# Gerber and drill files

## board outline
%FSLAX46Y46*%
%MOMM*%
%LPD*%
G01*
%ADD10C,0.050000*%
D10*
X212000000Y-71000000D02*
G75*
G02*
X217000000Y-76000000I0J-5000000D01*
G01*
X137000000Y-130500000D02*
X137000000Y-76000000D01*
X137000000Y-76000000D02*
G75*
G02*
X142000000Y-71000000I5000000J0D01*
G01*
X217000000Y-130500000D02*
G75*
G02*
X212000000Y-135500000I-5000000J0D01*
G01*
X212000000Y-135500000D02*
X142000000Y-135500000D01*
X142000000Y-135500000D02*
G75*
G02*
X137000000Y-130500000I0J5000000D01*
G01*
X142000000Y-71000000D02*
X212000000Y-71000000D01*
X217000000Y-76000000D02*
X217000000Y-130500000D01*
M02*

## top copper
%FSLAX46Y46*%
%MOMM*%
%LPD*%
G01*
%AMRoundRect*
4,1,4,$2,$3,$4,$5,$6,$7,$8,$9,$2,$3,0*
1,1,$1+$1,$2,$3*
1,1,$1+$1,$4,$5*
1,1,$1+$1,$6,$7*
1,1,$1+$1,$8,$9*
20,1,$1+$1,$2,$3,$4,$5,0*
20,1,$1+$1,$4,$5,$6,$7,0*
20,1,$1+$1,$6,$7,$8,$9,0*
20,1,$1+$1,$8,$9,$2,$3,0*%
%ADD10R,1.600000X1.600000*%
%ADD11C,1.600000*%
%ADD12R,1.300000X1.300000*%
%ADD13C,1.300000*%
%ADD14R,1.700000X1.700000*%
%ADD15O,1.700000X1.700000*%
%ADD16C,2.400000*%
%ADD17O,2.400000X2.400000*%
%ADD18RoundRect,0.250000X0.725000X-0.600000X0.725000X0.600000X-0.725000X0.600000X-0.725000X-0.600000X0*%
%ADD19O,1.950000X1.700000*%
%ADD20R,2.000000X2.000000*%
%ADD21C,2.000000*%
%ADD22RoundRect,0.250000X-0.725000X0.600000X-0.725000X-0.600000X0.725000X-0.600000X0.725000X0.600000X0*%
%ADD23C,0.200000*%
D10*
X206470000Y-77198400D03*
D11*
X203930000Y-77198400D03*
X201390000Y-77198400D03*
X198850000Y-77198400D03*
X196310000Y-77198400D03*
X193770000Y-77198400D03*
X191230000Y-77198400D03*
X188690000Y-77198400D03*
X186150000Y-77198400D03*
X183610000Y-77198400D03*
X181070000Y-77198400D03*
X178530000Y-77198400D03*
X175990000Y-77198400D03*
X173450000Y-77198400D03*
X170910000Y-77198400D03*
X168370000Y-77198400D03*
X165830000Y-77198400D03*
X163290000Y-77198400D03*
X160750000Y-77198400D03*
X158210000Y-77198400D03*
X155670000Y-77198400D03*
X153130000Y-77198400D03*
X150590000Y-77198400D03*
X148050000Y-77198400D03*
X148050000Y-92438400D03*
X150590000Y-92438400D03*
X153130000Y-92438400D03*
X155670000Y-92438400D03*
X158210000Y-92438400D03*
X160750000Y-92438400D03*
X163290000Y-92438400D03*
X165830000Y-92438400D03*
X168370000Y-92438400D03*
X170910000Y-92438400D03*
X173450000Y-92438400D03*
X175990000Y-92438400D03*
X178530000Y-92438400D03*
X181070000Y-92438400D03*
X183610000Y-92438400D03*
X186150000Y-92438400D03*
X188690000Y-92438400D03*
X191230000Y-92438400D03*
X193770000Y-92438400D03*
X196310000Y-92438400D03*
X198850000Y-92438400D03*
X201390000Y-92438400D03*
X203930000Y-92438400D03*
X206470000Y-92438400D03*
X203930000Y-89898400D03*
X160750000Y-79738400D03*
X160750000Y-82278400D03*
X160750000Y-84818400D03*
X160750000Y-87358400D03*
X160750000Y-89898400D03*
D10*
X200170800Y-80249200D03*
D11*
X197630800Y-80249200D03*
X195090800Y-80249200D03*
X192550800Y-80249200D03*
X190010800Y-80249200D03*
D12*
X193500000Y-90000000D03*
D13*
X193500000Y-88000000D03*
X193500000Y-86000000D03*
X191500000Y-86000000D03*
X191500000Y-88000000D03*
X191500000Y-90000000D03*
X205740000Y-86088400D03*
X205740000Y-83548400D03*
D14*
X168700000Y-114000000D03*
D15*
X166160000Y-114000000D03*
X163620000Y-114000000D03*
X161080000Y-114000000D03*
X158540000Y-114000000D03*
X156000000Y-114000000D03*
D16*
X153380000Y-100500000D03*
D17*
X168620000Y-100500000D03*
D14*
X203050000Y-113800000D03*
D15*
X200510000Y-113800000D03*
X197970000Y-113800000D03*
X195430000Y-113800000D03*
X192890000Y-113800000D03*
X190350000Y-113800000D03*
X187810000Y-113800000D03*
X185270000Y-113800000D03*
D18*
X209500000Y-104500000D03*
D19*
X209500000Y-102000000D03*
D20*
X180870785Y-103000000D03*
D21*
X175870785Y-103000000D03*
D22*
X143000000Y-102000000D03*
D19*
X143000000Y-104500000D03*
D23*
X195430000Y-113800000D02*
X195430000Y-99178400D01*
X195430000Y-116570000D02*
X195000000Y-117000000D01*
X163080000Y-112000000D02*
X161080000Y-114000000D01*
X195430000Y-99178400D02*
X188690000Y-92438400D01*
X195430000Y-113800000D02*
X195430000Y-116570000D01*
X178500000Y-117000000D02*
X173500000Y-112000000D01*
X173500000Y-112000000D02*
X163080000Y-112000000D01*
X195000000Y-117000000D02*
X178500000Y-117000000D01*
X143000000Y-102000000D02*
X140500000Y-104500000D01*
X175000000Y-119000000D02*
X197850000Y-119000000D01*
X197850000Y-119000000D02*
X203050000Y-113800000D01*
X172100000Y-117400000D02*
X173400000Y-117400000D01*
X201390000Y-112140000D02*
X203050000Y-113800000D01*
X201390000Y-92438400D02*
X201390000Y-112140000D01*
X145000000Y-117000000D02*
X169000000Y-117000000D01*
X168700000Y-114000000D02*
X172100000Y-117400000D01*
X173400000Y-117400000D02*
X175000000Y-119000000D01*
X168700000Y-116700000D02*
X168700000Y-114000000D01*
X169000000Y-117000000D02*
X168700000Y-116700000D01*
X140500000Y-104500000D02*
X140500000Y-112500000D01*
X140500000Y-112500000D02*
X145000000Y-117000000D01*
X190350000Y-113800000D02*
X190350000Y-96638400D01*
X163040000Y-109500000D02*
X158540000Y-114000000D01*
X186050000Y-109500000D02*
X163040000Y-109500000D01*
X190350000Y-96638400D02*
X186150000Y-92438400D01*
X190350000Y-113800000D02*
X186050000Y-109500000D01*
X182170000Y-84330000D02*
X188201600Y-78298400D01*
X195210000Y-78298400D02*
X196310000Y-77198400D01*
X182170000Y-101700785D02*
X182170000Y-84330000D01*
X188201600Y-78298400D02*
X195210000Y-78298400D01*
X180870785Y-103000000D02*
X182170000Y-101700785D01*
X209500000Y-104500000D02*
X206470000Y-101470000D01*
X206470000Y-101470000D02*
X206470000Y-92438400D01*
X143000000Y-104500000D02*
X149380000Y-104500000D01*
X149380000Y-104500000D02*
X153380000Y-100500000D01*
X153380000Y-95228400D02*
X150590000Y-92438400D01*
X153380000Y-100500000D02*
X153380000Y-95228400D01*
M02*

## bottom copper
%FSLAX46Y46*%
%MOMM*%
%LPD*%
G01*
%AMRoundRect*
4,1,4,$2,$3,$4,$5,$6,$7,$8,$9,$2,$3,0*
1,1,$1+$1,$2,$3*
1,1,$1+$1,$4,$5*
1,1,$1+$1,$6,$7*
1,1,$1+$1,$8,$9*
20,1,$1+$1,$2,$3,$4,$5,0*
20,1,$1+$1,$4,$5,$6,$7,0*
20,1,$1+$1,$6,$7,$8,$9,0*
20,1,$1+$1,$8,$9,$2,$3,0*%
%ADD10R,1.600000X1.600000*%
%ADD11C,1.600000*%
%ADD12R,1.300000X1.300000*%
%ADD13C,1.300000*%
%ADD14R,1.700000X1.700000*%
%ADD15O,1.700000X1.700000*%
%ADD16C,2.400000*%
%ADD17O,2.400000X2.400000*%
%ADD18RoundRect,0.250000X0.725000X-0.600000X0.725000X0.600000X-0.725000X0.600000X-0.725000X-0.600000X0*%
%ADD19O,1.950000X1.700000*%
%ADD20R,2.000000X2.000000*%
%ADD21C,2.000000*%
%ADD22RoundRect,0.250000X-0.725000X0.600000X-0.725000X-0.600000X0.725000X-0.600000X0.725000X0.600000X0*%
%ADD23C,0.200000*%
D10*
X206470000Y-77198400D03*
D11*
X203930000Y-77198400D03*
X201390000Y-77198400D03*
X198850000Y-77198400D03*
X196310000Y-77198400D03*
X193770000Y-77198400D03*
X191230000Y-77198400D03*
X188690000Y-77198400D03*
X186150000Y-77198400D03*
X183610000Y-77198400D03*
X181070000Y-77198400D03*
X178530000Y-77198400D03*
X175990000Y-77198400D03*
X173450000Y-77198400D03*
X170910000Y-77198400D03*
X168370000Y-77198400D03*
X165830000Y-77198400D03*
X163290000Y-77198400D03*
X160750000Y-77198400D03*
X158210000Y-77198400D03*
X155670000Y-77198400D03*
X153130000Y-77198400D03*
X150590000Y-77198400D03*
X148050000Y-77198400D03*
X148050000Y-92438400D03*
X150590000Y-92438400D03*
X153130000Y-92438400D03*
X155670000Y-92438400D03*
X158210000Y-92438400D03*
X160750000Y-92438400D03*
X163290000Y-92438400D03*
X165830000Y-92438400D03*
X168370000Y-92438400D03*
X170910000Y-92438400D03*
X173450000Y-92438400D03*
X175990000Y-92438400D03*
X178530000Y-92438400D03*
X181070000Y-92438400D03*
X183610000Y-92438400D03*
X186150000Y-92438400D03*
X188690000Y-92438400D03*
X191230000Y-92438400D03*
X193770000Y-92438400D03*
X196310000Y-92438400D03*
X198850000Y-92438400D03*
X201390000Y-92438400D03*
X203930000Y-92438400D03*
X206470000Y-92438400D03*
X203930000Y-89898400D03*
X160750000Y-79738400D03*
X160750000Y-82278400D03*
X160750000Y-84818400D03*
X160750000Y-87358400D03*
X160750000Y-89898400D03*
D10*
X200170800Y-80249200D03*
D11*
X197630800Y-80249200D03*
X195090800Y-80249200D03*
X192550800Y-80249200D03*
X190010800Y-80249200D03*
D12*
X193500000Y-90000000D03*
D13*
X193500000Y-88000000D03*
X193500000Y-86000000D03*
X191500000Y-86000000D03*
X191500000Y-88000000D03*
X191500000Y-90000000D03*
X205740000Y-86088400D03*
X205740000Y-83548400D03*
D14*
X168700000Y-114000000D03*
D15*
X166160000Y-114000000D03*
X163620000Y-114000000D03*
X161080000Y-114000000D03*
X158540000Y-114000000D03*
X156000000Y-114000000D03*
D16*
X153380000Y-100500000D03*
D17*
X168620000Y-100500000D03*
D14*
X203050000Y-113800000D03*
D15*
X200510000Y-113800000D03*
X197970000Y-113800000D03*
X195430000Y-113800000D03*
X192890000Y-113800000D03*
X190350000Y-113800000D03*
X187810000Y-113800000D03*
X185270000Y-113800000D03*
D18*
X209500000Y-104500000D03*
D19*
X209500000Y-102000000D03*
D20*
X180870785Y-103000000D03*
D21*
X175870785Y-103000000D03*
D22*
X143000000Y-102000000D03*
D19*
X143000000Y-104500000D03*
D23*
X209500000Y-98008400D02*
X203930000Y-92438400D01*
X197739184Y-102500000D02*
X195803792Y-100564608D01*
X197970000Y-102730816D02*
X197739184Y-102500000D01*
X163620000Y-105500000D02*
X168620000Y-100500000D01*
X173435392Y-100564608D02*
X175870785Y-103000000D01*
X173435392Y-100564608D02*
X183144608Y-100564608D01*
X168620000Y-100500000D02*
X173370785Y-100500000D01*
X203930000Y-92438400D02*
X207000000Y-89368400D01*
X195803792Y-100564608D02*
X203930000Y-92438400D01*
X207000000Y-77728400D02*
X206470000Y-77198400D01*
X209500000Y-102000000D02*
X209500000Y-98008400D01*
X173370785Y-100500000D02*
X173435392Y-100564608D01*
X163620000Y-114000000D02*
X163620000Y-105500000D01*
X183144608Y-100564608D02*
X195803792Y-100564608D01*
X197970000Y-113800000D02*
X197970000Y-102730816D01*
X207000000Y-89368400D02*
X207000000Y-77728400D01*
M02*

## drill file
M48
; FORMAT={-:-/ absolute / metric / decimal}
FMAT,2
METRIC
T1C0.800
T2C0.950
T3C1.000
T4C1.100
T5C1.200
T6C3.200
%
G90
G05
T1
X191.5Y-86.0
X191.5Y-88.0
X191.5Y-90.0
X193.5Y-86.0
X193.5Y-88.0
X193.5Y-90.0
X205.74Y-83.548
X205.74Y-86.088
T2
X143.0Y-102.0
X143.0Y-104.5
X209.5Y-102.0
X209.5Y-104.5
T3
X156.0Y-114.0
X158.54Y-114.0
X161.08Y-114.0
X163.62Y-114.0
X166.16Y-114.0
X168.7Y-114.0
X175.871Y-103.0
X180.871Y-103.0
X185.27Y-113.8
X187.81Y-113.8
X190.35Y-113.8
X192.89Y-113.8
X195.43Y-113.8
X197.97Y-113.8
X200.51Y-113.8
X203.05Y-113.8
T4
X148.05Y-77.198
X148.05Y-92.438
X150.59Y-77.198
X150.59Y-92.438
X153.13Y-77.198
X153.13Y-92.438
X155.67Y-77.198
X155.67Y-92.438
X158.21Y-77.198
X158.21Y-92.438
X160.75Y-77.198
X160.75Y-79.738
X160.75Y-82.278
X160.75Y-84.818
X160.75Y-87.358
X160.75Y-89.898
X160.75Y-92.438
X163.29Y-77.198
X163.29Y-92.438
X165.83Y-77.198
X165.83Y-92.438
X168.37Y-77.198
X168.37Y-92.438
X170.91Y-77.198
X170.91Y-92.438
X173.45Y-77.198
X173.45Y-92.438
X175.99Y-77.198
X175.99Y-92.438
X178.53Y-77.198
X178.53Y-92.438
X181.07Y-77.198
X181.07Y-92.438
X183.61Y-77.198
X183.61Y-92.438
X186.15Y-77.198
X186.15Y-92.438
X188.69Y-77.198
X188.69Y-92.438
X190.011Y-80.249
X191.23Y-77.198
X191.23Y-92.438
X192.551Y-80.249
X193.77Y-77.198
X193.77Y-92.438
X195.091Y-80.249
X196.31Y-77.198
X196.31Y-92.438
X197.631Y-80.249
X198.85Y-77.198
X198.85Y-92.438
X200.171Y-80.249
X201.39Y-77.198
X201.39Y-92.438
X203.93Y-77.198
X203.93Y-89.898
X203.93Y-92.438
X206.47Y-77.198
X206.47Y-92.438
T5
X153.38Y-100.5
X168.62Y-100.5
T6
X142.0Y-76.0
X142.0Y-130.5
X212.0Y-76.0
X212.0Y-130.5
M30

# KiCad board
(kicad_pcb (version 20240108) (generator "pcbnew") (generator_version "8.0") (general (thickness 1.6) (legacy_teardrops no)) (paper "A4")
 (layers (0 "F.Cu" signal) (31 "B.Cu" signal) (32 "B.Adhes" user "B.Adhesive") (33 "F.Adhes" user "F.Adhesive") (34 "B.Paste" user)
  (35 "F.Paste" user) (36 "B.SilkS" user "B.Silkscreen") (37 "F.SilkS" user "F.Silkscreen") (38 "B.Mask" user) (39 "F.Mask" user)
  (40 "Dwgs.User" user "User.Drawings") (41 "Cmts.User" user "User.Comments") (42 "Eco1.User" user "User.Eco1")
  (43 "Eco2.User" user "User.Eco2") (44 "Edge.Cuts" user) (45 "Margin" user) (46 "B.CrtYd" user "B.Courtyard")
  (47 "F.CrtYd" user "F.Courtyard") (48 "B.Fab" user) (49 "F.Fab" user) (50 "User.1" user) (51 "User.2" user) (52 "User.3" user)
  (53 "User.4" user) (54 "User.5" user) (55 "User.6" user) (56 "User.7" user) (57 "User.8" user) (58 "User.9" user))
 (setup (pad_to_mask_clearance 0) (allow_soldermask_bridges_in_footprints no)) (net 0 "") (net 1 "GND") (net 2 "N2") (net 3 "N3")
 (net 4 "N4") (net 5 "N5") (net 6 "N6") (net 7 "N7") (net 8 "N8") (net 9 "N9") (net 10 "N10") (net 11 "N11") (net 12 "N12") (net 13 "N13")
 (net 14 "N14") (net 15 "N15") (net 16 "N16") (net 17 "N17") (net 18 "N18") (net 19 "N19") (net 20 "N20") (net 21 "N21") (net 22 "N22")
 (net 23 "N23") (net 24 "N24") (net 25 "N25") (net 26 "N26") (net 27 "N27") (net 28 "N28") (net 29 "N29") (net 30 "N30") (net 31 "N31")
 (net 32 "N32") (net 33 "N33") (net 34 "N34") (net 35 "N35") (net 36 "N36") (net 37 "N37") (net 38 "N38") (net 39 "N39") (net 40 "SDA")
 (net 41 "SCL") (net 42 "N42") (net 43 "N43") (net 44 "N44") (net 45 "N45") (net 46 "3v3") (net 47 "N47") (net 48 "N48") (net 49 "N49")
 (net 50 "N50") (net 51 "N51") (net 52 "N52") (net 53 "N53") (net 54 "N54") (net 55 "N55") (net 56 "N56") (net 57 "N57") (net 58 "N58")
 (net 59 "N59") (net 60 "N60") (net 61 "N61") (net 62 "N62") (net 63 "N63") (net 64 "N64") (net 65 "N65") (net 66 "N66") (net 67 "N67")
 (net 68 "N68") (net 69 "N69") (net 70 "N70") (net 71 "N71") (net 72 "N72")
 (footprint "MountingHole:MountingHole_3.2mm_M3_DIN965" (layer "F.Cu") (at 212 76)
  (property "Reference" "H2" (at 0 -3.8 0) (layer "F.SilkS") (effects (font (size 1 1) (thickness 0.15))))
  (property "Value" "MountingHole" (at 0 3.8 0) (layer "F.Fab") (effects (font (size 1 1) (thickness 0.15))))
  (pad "" np_thru_hole circle (at 0 0) (size 3.2 3.2) (drill 3.2) (layers "*.Cu" "*.Mask")))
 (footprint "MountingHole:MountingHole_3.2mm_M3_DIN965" (layer "F.Cu") (at 142 76)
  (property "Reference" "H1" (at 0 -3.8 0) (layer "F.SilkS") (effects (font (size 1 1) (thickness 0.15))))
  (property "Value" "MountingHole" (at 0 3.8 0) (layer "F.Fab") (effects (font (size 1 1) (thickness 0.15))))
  (pad "" np_thru_hole circle (at 0 0) (size 3.2 3.2) (drill 3.2) (layers "*.Cu" "*.Mask")))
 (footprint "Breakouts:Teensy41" (layer "F.Cu") (at 177.26 84.8184 180)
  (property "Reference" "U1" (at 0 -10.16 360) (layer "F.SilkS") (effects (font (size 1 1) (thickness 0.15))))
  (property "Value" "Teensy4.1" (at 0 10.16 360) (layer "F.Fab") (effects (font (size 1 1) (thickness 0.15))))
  (pad "1" thru_hole rect (at -29.21 7.62 180) (size 1.6 1.6) (drill 1.1) (layers "*.Cu" "*.Mask") (remove_unused_layers no) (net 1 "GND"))
  (pad "2" thru_hole circle (at -26.67 7.62 180) (size 1.6 1.6) (drill 1.1) (layers "*.Cu" "*.Mask") (remove_unused_layers no) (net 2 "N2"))
  (pad "3" thru_hole circle (at -24.13 7.62 180) (size 1.6 1.6) (drill 1.1) (layers "*.Cu" "*.Mask") (remove_unused_layers no) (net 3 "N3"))
  (pad "4" thru_hole circle (at -21.59 7.62 180) (size 1.6 1.6) (drill 1.1) (layers "*.Cu" "*.Mask") (remove_unused_layers no) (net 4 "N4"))
  (pad "5" thru_hole circle (at -19.05 7.62 180) (size 1.6 1.6) (drill 1.1) (layers "*.Cu" "*.Mask") (remove_unused_layers no) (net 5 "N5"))
  (pad "6" thru_hole circle (at -16.51 7.62 180) (size 1.6 1.6) (drill 1.1) (layers "*.Cu" "*.Mask") (remove_unused_layers no) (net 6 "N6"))
  (pad "7" thru_hole circle (at -13.97 7.62 180) (size 1.6 1.6) (drill 1.1) (layers "*.Cu" "*.Mask") (remove_unused_layers no) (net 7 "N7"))
  (pad "8" thru_hole circle (at -11.43 7.62 180) (size 1.6 1.6) (drill 1.1) (layers "*.Cu" "*.Mask") (remove_unused_layers no) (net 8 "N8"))
  (pad "9" thru_hole circle (at -8.89 7.62 180) (size 1.6 1.6) (drill 1.1) (layers "*.Cu" "*.Mask") (remove_unused_layers no) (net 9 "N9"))
  (pad "10" thru_hole circle (at -6.35 7.62 180) (size 1.6 1.6) (drill 1.1) (layers "*.Cu" "*.Mask") (remove_unused_layers no)
   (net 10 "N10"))
  (pad "11" thru_hole circle (at -3.81 7.62 180) (size 1.6 1.6) (drill 1.1) (layers "*.Cu" "*.Mask") (remove_unused_layers no)
   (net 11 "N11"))
  (pad "12" thru_hole circle (at -1.27 7.62 180) (size 1.6 1.6) (drill 1.1) (layers "*.Cu" "*.Mask") (remove_unused_layers no)
   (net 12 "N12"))
  (pad "13" thru_hole circle (at 1.27 7.62 180) (size 1.6 1.6) (drill 1.1) (layers "*.Cu" "*.Mask") (remove_unused_layers no) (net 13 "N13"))
  (pad "14" thru_hole circle (at 3.81 7.62 180) (size 1.6 1.6) (drill 1.1) (layers "*.Cu" "*.Mask") (remove_unused_layers no) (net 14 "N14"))
  (pad "15" thru_hole circle (at 6.35 7.62 180) (size 1.6 1.6) (drill 1.1) (layers "*.Cu" "*.Mask") (remove_unused_layers no) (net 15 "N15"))
  (pad "16" thru_hole circle (at 8.89 7.62 180) (size 1.6 1.6) (drill 1.1) (layers "*.Cu" "*.Mask") (remove_unused_layers no) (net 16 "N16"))
  (pad "17" thru_hole circle (at 11.43 7.62 180) (size 1.6 1.6) (drill 1.1) (layers "*.Cu" "*.Mask") (remove_unused_layers no)
   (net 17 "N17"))
  (pad "18" thru_hole circle (at 13.97 7.62 180) (size 1.6 1.6) (drill 1.1) (layers "*.Cu" "*.Mask") (remove_unused_layers no)
   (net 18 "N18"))
  (pad "19" thru_hole circle (at 16.51 7.62 180) (size 1.6 1.6) (drill 1.1) (layers "*.Cu" "*.Mask") (remove_unused_layers no)
   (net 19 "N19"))
  (pad "20" thru_hole circle (at 19.05 7.62 180) (size 1.6 1.6) (drill 1.1) (layers "*.Cu" "*.Mask") (remove_unused_layers no)
   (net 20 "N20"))
  (pad "21" thru_hole circle (at 21.59 7.62 180) (size 1.6 1.6) (drill 1.1) (layers "*.Cu" "*.Mask") (remove_unused_layers no)
   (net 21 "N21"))
  (pad "22" thru_hole circle (at 24.13 7.62 180) (size 1.6 1.6) (drill 1.1) (layers "*.Cu" "*.Mask") (remove_unused_layers no)
   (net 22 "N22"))
  (pad "23" thru_hole circle (at 26.67 7.62 180) (size 1.6 1.6) (drill 1.1) (layers "*.Cu" "*.Mask") (remove_unused_layers no)
   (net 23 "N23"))
  (pad "24" thru_hole circle (at 29.21 7.62 180) (size 1.6 1.6) (drill 1.1) (layers "*.Cu" "*.Mask") (remove_unused_layers no)
   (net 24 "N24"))
  (pad "25" thru_hole circle (at 29.21 -7.62 180) (size 1.6 1.6) (drill 1.1) (layers "*.Cu" "*.Mask") (remove_unused_layers no)
   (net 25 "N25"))
  (pad "26" thru_hole circle (at 26.67 -7.62 180) (size 1.6 1.6) (drill 1.1) (layers "*.Cu" "*.Mask") (remove_unused_layers no)
   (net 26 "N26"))
  (pad "27" thru_hole circle (at 24.13 -7.62 180) (size 1.6 1.6) (drill 1.1) (layers "*.Cu" "*.Mask") (remove_unused_layers no)
   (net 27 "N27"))
  (pad "28" thru_hole circle (at 21.59 -7.62 180) (size 1.6 1.6) (drill 1.1) (layers "*.Cu" "*.Mask") (remove_unused_layers no)
   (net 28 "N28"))
  (pad "29" thru_hole circle (at 19.05 -7.62 180) (size 1.6 1.6) (drill 1.1) (layers "*.Cu" "*.Mask") (remove_unused_layers no)
   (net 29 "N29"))
  (pad "30" thru_hole circle (at 16.51 -7.62 180) (size 1.6 1.6) (drill 1.1) (layers "*.Cu" "*.Mask") (remove_unused_layers no)
   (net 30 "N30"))
  (pad "31" thru_hole circle (at 13.97 -7.62 180) (size 1.6 1.6) (drill 1.1) (layers "*.Cu" "*.Mask") (remove_unused_layers no)
   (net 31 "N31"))
  (pad "32" thru_hole circle (at 11.43 -7.62 180) (size 1.6 1.6) (drill 1.1) (layers "*.Cu" "*.Mask") (remove_unused_layers no)
   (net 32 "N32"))
  (pad "33" thru_hole circle (at 8.89 -7.62 180) (size 1.6 1.6) (drill 1.1) (layers "*.Cu" "*.Mask") (remove_unused_layers no)
   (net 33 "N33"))
  (pad "34" thru_hole circle (at 6.35 -7.62 180) (size 1.6 1.6) (drill 1.1) (layers "*.Cu" "*.Mask") (remove_unused_layers no)
   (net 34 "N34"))
  (pad "35" thru_hole circle (at 3.81 -7.62 180) (size 1.6 1.6) (drill 1.1) (layers "*.Cu" "*.Mask") (remove_unused_layers no)
   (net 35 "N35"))
  (pad "36" thru_hole circle (at 1.27 -7.62 180) (size 1.6 1.6) (drill 1.1) (layers "*.Cu" "*.Mask") (remove_unused_layers no)
   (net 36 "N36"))
  (pad "37" thru_hole circle (at -1.27 -7.62 180) (size 1.6 1.6) (drill 1.1) (layers "*.Cu" "*.Mask") (remove_unused_layers no)
   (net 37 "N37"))
  (pad "38" thru_hole circle (at -3.81 -7.62 180) (size 1.6 1.6) (drill 1.1) (layers "*.Cu" "*.Mask") (remove_unused_layers no)
   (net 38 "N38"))
  (pad "39" thru_hole circle (at -6.35 -7.62 180) (size 1.6 1.6) (drill 1.1) (layers "*.Cu" "*.Mask") (remove_unused_layers no)
   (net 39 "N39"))
  (pad "40" thru_hole circle (at -8.89 -7.62 180) (size 1.6 1.6) (drill 1.1) (layers "*.Cu" "*.Mask") (remove_unused_layers no)
   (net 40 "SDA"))
  (pad "41" thru_hole circle (at -11.43 -7.62 180) (size 1.6 1.6) (drill 1.1) (layers "*.Cu" "*.Mask") (remove_unused_layers no)
   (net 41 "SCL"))
  (pad "42" thru_hole circle (at -13.97 -7.62 180) (size 1.6 1.6) (drill 1.1) (layers "*.Cu" "*.Mask") (remove_unused_layers no)
   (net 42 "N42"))
  (pad "43" thru_hole circle (at -16.51 -7.62 180) (size 1.6 1.6) (drill 1.1) (layers "*.Cu" "*.Mask") (remove_unused_layers no)
   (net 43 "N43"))
  (pad "44" thru_hole circle (at -19.05 -7.62 180) (size 1.6 1.6) (drill 1.1) (layers "*.Cu" "*.Mask") (remove_unused_layers no)
   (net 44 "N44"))
  (pad "45" thru_hole circle (at -21.59 -7.62 180) (size 1.6 1.6) (drill 1.1) (layers "*.Cu" "*.Mask") (remove_unused_layers no)
   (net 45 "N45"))
  (pad "46" thru_hole circle (at -24.13 -7.62 180) (size 1.6 1.6) (drill 1.1) (layers "*.Cu" "*.Mask") (remove_unused_layers no)
   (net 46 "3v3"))
  (pad "47" thru_hole circle (at -26.67 -7.62 180) (size 1.6 1.6) (drill 1.1) (layers "*.Cu" "*.Mask") (remove_unused_layers no)
   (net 1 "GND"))
  (pad "48" thru_hole circle (at -29.21 -7.62 180) (size 1.6 1.6) (drill 1.1) (layers "*.Cu" "*.Mask") (remove_unused_layers no)
   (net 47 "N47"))
  (pad "49" thru_hole circle (at -26.67 -5.08 180) (size 1.6 1.6) (drill 1.1) (layers "*.Cu" "*.Mask") (remove_unused_layers no)
   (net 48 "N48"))
  (pad "50" thru_hole circle (at 16.51 5.08 180) (size 1.6 1.6) (drill 1.1) (layers "*.Cu" "*.Mask") (remove_unused_layers no)
   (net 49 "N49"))
  (pad "51" thru_hole circle (at 16.51 2.54 180) (size 1.6 1.6) (drill 1.1) (layers "*.Cu" "*.Mask") (remove_unused_layers no)
   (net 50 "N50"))
  (pad "52" thru_hole circle (at 16.51 0 180) (size 1.6 1.6) (drill 1.1) (layers "*.Cu" "*.Mask") (remove_unused_layers no) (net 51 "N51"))
  (pad "53" thru_hole circle (at 16.51 -2.54 180) (size 1.6 1.6) (drill 1.1) (layers "*.Cu" "*.Mask") (remove_unused_layers no)
   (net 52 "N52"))
  (pad "54" thru_hole circle (at 16.51 -5.08 180) (size 1.6 1.6) (drill 1.1) (layers "*.Cu" "*.Mask") (remove_unused_layers no)
   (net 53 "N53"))
  (pad "55" thru_hole rect (at -22.9108 4.5692 180) (size 1.6 1.6) (drill 1.1) (layers "*.Cu" "*.Mask") (remove_unused_layers no)
   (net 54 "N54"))
  (pad "56" thru_hole circle (at -20.3708 4.5692 180) (size 1.6 1.6) (drill 1.1) (layers "*.Cu" "*.Mask") (remove_unused_layers no)
   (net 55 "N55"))
  (pad "57" thru_hole circle (at -17.8308 4.5692 180) (size 1.6 1.6) (drill 1.1) (layers "*.Cu" "*.Mask") (remove_unused_layers no)
   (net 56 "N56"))
  (pad "58" thru_hole circle (at -15.2908 4.5692 180) (size 1.6 1.6) (drill 1.1) (layers "*.Cu" "*.Mask") (remove_unused_layers no)
   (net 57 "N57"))
  (pad "59" thru_hole circle (at -12.7508 4.5692 180) (size 1.6 1.6) (drill 1.1) (layers "*.Cu" "*.Mask") (remove_unused_layers no)
   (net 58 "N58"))
  (pad "60" thru_hole rect (at -16.24 -5.1816 180) (size 1.3 1.3) (drill 0.8) (layers "*.Cu" "*.Mask") (remove_unused_layers no)
   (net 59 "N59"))
  (pad "61" thru_hole circle (at -16.24 -3.1816 180) (size 1.3 1.3) (drill 0.8) (layers "*.Cu" "*.Mask") (remove_unused_layers no)
   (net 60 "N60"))
  (pad "62" thru_hole circle (at -16.24 -1.1816 180) (size 1.3 1.3) (drill 0.8) (layers "*.Cu" "*.Mask") (remove_unused_layers no)
   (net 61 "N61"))
  (pad "63" thru_hole circle (at -14.24 -1.1816 180) (size 1.3 1.3) (drill 0.8) (layers "*.Cu" "*.Mask") (remove_unused_layers no)
   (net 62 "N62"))
  (pad "64" thru_hole circle (at -14.24 -3.1816 180) (size 1.3 1.3) (drill 0.8) (layers "*.Cu" "*.Mask") (remove_unused_layers no)
   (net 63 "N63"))
  (pad "65" thru_hole circle (at -14.24 -5.1816 180) (size 1.3 1.3) (drill 0.8) (layers "*.Cu" "*.Mask") (remove_unused_layers no)
   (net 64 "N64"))
  (pad "66" thru_hole circle (at -28.48 -1.27 180) (size 1.3 1.3) (drill 0.8) (layers "*.Cu" "*.Mask") (remove_unused_layers no)
   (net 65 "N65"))
  (pad "67" thru_hole circle (at -28.48 1.27 180) (size 1.3 1.3) (drill 0.8) (layers "*.Cu" "*.Mask") (remove_unused_layers no)
   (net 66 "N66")))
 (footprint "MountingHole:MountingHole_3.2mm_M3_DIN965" (layer "F.Cu") (at 212 130.5)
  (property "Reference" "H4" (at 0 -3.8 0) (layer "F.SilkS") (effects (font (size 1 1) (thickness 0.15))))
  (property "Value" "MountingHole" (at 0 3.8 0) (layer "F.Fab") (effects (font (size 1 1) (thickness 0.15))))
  (pad "" np_thru_hole circle (at 0 0) (size 3.2 3.2) (drill 3.2) (layers "*.Cu" "*.Mask")))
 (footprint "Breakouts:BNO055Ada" (layer "F.Cu") (at 162.5 121 180)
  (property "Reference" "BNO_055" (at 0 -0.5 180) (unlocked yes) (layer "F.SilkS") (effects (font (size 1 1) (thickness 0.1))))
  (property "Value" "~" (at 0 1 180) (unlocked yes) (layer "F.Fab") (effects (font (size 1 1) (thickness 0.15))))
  (pad "1" thru_hole rect (at -6.2 7 270) (size 1.7 1.7) (drill 1) (layers "*.Cu" "*.Mask") (remove_unused_layers no) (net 46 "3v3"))
  (pad "2" thru_hole oval (at -3.66 7 270) (size 1.7 1.7) (drill 1) (layers "*.Cu" "*.Mask") (remove_unused_layers no) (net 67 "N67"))
  (pad "3" thru_hole oval (at -1.12 7 270) (size 1.7 1.7) (drill 1) (layers "*.Cu" "*.Mask") (remove_unused_layers no) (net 1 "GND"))
  (pad "4" thru_hole oval (at 1.42 7 270) (size 1.7 1.7) (drill 1) (layers "*.Cu" "*.Mask") (remove_unused_layers no) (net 41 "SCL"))
  (pad "5" thru_hole oval (at 3.96 7 270) (size 1.7 1.7) (drill 1) (layers "*.Cu" "*.Mask") (remove_unused_layers no) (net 40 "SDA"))
  (pad "6" thru_hole oval (at 6.5 7 270) (size 1.7 1.7) (drill 1) (layers "*.Cu" "*.Mask") (remove_unused_layers no) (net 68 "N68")))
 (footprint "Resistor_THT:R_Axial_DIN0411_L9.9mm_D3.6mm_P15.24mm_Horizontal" (layer "F.Cu") (at 153.38 100.5)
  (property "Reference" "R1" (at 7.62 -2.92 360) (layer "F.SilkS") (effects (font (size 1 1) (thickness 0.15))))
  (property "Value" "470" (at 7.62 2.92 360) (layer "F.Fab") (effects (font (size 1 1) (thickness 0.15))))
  (pad "1" thru_hole circle (at 0 0) (size 2.4 2.4) (drill 1.2) (layers "*.Cu" "*.Mask") (remove_unused_layers no) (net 26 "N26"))
  (pad "2" thru_hole oval (at 15.24 0) (size 2.4 2.4) (drill 1.2) (layers "*.Cu" "*.Mask") (remove_unused_layers no) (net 1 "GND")))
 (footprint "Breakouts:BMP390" (layer "F.Cu") (at 194 121 180)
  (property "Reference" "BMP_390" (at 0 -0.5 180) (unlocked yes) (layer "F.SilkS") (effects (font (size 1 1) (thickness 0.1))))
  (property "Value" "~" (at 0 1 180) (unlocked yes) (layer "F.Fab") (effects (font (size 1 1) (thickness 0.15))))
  (pad "1" thru_hole rect (at -9.05 7.2 270) (size 1.7 1.7) (drill 1) (layers "*.Cu" "*.Mask") (remove_unused_layers no) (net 46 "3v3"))
  (pad "2" thru_hole oval (at -6.51 7.2 270) (size 1.7 1.7) (drill 1) (layers "*.Cu" "*.Mask") (remove_unused_layers no) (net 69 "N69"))
  (pad "3" thru_hole oval (at -3.97 7.2 270) (size 1.7 1.7) (drill 1) (layers "*.Cu" "*.Mask") (remove_unused_layers no) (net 1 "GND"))
  (pad "4" thru_hole oval (at -1.43 7.2 270) (size 1.7 1.7) (drill 1) (layers "*.Cu" "*.Mask") (remove_unused_layers no) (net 41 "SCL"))
  (pad "5" thru_hole oval (at 1.11 7.2 270) (size 1.7 1.7) (drill 1) (layers "*.Cu" "*.Mask") (remove_unused_layers no) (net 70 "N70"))
  (pad "6" thru_hole oval (at 3.65 7.2 270) (size 1.7 1.7) (drill 1) (layers "*.Cu" "*.Mask") (remove_unused_layers no) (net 40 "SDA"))
  (pad "7" thru_hole oval (at 6.19 7.2 270) (size 1.7 1.7) (drill 1) (layers "*.Cu" "*.Mask") (remove_unused_layers no) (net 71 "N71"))
  (pad "8" thru_hole oval (at 8.73 7.2 270) (size 1.7 1.7) (drill 1) (layers "*.Cu" "*.Mask") (remove_unused_layers no) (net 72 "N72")))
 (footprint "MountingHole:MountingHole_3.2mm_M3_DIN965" (layer "F.Cu") (at 142 130.5)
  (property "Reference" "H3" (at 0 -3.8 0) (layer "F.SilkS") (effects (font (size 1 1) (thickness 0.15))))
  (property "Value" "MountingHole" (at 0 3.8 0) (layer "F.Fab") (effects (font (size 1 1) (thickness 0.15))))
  (pad "" np_thru_hole circle (at 0 0) (size 3.2 3.2) (drill 3.2) (layers "*.Cu" "*.Mask")))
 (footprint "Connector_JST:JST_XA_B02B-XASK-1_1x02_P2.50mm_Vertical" (layer "F.Cu") (at 209.5 104.5 90)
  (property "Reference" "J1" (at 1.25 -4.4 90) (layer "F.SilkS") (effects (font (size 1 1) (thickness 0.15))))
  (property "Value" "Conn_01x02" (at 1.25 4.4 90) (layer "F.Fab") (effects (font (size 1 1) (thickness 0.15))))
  (pad "1" thru_hole roundrect (at 0 0 90) (size 1.7 1.95) (drill 0.95) (layers "*.Cu" "*.Mask") (remove_unused_layers no)
   (roundrect_rratio 0.147059) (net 47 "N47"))
  (pad "2" thru_hole oval (at 2.5 0 90) (size 1.7 1.95) (drill 0.95) (layers "*.Cu" "*.Mask") (remove_unused_layers no) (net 1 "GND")))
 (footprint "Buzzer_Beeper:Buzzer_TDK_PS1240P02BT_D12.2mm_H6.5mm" (layer "F.Cu") (at 180.870785 103 180)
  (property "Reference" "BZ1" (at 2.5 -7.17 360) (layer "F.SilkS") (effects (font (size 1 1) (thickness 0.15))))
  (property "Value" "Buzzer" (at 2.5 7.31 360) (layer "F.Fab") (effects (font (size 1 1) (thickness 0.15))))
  (pad "1" thru_hole rect (at 0 0 180) (size 2 2) (drill 1) (layers "*.Cu" "*.Mask") (remove_unused_layers no) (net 5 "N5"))
  (pad "2" thru_hole circle (at 5 0 180) (size 2 2) (drill 1) (layers "*.Cu" "*.Mask") (remove_unused_layers no) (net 1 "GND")))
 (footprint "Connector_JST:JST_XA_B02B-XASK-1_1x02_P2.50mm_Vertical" (layer "F.Cu") (at 143 102 -90)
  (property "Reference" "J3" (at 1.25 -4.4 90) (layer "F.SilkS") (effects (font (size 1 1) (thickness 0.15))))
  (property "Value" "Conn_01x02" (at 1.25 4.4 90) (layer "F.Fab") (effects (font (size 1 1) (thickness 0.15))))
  (pad "1" thru_hole roundrect (at 0 0 270) (size 1.7 1.95) (drill 0.95) (layers "*.Cu" "*.Mask") (remove_unused_layers no)
   (roundrect_rratio 0.147059) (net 46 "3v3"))
  (pad "2" thru_hole oval (at 2.5 0 270) (size 1.7 1.95) (drill 0.95) (layers "*.Cu" "*.Mask") (remove_unused_layers no) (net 26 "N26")))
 (gr_arc (start 212 71) (mid 215.535534 72.464466) (end 217 76) (stroke (width 0.05) (type default)) (layer "Edge.Cuts"))
 (gr_line (start 137 130.5) (end 137 76) (stroke (width 0.05) (type default)) (layer "Edge.Cuts"))
 (gr_arc (start 137 76) (mid 138.464466 72.464466) (end 142 71) (stroke (width 0.05) (type default)) (layer "Edge.Cuts"))
 (gr_arc (start 217 130.5) (mid 215.535534 134.035534) (end 212 135.5) (stroke (width 0.05) (type default)) (layer "Edge.Cuts"))
 (gr_line (start 212 135.5) (end 142 135.5) (stroke (width 0.05) (type default)) (layer "Edge.Cuts"))
 (gr_arc (start 142 135.5) (mid 138.464466 134.035534) (end 137 130.5) (stroke (width 0.05) (type default)) (layer "Edge.Cuts"))
 (gr_line (start 142 71) (end 212 71) (stroke (width 0.05) (type default)) (layer "Edge.Cuts"))
 (gr_line (start 217 76) (end 217 130.5) (stroke (width 0.05) (type default)) (layer "Edge.Cuts"))
 (segment (start 195.43 113.8) (end 195.43 99.1784) (width 0.2) (layer "F.Cu") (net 41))
 (segment (start 195.43 116.57) (end 195 117) (width 0.2) (layer "F.Cu") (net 41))
 (segment (start 163.08 112) (end 161.08 114) (width 0.2) (layer "F.Cu") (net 41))
 (segment (start 195.43 99.1784) (end 188.69 92.4384) (width 0.2) (layer "F.Cu") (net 41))
 (segment (start 195.43 113.8) (end 195.43 116.57) (width 0.2) (layer "F.Cu") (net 41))
 (segment (start 178.5 117) (end 173.5 112) (width 0.2) (layer "F.Cu") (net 41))
 (segment (start 173.5 112) (end 163.08 112) (width 0.2) (layer "F.Cu") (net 41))
 (segment (start 195 117) (end 178.5 117) (width 0.2) (layer "F.Cu") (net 41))
 (segment (start 143 102) (end 140.5 104.5) (width 0.2) (layer "F.Cu") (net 46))
 (segment (start 175 119) (end 197.85 119) (width 0.2) (layer "F.Cu") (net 46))
 (segment (start 197.85 119) (end 203.05 113.8) (width 0.2) (layer "F.Cu") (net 46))
 (segment (start 172.1 117.4) (end 173.4 117.4) (width 0.2) (layer "F.Cu") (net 46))
 (segment (start 201.39 112.14) (end 203.05 113.8) (width 0.2) (layer "F.Cu") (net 46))
 (segment (start 201.39 92.4384) (end 201.39 112.14) (width 0.2) (layer "F.Cu") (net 46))
 (segment (start 145 117) (end 169 117) (width 0.2) (layer "F.Cu") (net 46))
 (segment (start 168.7 114) (end 172.1 117.4) (width 0.2) (layer "F.Cu") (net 46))
 (segment (start 173.4 117.4) (end 175 119) (width 0.2) (layer "F.Cu") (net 46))
 (segment (start 168.7 116.7) (end 168.7 114) (width 0.2) (layer "F.Cu") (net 46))
 (segment (start 169 117) (end 168.7 116.7) (width 0.2) (layer "F.Cu") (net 46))
 (segment (start 140.5 104.5) (end 140.5 112.5) (width 0.2) (layer "F.Cu") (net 46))
 (segment (start 140.5 112.5) (end 145 117) (width 0.2) (layer "F.Cu") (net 46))
 (segment (start 190.35 113.8) (end 190.35 96.6384) (width 0.2) (layer "F.Cu") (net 40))
 (segment (start 163.04 109.5) (end 158.54 114) (width 0.2) (layer "F.Cu") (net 40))
 (segment (start 186.05 109.5) (end 163.04 109.5) (width 0.2) (layer "F.Cu") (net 40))
 (segment (start 190.35 96.6384) (end 186.15 92.4384) (width 0.2) (layer "F.Cu") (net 40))
 (segment (start 190.35 113.8) (end 186.05 109.5) (width 0.2) (layer "F.Cu") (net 40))
 (segment (start 209.5 98.0084) (end 203.93 92.4384) (width 0.2) (layer "B.Cu") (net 1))
 (segment (start 197.739184 102.5) (end 195.803792 100.564608) (width 0.2) (layer "B.Cu") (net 1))
 (segment (start 197.97 102.730816) (end 197.739184 102.5) (width 0.2) (layer "B.Cu") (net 1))
 (segment (start 163.62 105.5) (end 168.62 100.5) (width 0.2) (layer "B.Cu") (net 1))
 (segment (start 173.435392 100.564608) (end 175.870785 103) (width 0.2) (layer "B.Cu") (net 1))
 (segment (start 173.435392 100.564608) (end 183.144608 100.564608) (width 0.2) (layer "B.Cu") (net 1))
 (segment (start 168.62 100.5) (end 173.370785 100.5) (width 0.2) (layer "B.Cu") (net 1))
 (segment (start 203.93 92.4384) (end 207 89.3684) (width 0.2) (layer "B.Cu") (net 1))
 (segment (start 195.803792 100.564608) (end 203.93 92.4384) (width 0.2) (layer "B.Cu") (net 1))
 (segment (start 207 77.7284) (end 206.47 77.1984) (width 0.2) (layer "B.Cu") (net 1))
 (segment (start 209.5 102) (end 209.5 98.0084) (width 0.2) (layer "B.Cu") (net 1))
 (segment (start 173.370785 100.5) (end 173.435392 100.564608) (width 0.2) (layer "B.Cu") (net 1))
 (segment (start 163.62 114) (end 163.62 105.5) (width 0.2) (layer "B.Cu") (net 1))
 (segment (start 183.144608 100.564608) (end 195.803792 100.564608) (width 0.2) (layer "B.Cu") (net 1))
 (segment (start 197.97 113.8) (end 197.97 102.730816) (width 0.2) (layer "B.Cu") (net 1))
 (segment (start 207 89.3684) (end 207 77.7284) (width 0.2) (layer "B.Cu") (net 1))
 (segment (start 182.17 84.33) (end 188.2016 78.2984) (width 0.2) (layer "F.Cu") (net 5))
 (segment (start 195.21 78.2984) (end 196.31 77.1984) (width 0.2) (layer "F.Cu") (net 5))
 (segment (start 182.17 101.700785) (end 182.17 84.33) (width 0.2) (layer "F.Cu") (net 5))
 (segment (start 188.2016 78.2984) (end 195.21 78.2984) (width 0.2) (layer "F.Cu") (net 5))
 (segment (start 180.870785 103) (end 182.17 101.700785) (width 0.2) (layer "F.Cu") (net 5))
 (segment (start 209.5 104.5) (end 206.47 101.47) (width 0.2) (layer "F.Cu") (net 47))
 (segment (start 206.47 101.47) (end 206.47 92.4384) (width 0.2) (layer "F.Cu") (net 47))
 (segment (start 143 104.5) (end 149.38 104.5) (width 0.2) (layer "F.Cu") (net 26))
 (segment (start 149.38 104.5) (end 153.38 100.5) (width 0.2) (layer "F.Cu") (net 26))
 (segment (start 153.38 95.2284) (end 150.59 92.4384) (width 0.2) (layer "F.Cu") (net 26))
 (segment (start 153.38 100.5) (end 153.38 95.2284) (width 0.2) (layer "F.Cu") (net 26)))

